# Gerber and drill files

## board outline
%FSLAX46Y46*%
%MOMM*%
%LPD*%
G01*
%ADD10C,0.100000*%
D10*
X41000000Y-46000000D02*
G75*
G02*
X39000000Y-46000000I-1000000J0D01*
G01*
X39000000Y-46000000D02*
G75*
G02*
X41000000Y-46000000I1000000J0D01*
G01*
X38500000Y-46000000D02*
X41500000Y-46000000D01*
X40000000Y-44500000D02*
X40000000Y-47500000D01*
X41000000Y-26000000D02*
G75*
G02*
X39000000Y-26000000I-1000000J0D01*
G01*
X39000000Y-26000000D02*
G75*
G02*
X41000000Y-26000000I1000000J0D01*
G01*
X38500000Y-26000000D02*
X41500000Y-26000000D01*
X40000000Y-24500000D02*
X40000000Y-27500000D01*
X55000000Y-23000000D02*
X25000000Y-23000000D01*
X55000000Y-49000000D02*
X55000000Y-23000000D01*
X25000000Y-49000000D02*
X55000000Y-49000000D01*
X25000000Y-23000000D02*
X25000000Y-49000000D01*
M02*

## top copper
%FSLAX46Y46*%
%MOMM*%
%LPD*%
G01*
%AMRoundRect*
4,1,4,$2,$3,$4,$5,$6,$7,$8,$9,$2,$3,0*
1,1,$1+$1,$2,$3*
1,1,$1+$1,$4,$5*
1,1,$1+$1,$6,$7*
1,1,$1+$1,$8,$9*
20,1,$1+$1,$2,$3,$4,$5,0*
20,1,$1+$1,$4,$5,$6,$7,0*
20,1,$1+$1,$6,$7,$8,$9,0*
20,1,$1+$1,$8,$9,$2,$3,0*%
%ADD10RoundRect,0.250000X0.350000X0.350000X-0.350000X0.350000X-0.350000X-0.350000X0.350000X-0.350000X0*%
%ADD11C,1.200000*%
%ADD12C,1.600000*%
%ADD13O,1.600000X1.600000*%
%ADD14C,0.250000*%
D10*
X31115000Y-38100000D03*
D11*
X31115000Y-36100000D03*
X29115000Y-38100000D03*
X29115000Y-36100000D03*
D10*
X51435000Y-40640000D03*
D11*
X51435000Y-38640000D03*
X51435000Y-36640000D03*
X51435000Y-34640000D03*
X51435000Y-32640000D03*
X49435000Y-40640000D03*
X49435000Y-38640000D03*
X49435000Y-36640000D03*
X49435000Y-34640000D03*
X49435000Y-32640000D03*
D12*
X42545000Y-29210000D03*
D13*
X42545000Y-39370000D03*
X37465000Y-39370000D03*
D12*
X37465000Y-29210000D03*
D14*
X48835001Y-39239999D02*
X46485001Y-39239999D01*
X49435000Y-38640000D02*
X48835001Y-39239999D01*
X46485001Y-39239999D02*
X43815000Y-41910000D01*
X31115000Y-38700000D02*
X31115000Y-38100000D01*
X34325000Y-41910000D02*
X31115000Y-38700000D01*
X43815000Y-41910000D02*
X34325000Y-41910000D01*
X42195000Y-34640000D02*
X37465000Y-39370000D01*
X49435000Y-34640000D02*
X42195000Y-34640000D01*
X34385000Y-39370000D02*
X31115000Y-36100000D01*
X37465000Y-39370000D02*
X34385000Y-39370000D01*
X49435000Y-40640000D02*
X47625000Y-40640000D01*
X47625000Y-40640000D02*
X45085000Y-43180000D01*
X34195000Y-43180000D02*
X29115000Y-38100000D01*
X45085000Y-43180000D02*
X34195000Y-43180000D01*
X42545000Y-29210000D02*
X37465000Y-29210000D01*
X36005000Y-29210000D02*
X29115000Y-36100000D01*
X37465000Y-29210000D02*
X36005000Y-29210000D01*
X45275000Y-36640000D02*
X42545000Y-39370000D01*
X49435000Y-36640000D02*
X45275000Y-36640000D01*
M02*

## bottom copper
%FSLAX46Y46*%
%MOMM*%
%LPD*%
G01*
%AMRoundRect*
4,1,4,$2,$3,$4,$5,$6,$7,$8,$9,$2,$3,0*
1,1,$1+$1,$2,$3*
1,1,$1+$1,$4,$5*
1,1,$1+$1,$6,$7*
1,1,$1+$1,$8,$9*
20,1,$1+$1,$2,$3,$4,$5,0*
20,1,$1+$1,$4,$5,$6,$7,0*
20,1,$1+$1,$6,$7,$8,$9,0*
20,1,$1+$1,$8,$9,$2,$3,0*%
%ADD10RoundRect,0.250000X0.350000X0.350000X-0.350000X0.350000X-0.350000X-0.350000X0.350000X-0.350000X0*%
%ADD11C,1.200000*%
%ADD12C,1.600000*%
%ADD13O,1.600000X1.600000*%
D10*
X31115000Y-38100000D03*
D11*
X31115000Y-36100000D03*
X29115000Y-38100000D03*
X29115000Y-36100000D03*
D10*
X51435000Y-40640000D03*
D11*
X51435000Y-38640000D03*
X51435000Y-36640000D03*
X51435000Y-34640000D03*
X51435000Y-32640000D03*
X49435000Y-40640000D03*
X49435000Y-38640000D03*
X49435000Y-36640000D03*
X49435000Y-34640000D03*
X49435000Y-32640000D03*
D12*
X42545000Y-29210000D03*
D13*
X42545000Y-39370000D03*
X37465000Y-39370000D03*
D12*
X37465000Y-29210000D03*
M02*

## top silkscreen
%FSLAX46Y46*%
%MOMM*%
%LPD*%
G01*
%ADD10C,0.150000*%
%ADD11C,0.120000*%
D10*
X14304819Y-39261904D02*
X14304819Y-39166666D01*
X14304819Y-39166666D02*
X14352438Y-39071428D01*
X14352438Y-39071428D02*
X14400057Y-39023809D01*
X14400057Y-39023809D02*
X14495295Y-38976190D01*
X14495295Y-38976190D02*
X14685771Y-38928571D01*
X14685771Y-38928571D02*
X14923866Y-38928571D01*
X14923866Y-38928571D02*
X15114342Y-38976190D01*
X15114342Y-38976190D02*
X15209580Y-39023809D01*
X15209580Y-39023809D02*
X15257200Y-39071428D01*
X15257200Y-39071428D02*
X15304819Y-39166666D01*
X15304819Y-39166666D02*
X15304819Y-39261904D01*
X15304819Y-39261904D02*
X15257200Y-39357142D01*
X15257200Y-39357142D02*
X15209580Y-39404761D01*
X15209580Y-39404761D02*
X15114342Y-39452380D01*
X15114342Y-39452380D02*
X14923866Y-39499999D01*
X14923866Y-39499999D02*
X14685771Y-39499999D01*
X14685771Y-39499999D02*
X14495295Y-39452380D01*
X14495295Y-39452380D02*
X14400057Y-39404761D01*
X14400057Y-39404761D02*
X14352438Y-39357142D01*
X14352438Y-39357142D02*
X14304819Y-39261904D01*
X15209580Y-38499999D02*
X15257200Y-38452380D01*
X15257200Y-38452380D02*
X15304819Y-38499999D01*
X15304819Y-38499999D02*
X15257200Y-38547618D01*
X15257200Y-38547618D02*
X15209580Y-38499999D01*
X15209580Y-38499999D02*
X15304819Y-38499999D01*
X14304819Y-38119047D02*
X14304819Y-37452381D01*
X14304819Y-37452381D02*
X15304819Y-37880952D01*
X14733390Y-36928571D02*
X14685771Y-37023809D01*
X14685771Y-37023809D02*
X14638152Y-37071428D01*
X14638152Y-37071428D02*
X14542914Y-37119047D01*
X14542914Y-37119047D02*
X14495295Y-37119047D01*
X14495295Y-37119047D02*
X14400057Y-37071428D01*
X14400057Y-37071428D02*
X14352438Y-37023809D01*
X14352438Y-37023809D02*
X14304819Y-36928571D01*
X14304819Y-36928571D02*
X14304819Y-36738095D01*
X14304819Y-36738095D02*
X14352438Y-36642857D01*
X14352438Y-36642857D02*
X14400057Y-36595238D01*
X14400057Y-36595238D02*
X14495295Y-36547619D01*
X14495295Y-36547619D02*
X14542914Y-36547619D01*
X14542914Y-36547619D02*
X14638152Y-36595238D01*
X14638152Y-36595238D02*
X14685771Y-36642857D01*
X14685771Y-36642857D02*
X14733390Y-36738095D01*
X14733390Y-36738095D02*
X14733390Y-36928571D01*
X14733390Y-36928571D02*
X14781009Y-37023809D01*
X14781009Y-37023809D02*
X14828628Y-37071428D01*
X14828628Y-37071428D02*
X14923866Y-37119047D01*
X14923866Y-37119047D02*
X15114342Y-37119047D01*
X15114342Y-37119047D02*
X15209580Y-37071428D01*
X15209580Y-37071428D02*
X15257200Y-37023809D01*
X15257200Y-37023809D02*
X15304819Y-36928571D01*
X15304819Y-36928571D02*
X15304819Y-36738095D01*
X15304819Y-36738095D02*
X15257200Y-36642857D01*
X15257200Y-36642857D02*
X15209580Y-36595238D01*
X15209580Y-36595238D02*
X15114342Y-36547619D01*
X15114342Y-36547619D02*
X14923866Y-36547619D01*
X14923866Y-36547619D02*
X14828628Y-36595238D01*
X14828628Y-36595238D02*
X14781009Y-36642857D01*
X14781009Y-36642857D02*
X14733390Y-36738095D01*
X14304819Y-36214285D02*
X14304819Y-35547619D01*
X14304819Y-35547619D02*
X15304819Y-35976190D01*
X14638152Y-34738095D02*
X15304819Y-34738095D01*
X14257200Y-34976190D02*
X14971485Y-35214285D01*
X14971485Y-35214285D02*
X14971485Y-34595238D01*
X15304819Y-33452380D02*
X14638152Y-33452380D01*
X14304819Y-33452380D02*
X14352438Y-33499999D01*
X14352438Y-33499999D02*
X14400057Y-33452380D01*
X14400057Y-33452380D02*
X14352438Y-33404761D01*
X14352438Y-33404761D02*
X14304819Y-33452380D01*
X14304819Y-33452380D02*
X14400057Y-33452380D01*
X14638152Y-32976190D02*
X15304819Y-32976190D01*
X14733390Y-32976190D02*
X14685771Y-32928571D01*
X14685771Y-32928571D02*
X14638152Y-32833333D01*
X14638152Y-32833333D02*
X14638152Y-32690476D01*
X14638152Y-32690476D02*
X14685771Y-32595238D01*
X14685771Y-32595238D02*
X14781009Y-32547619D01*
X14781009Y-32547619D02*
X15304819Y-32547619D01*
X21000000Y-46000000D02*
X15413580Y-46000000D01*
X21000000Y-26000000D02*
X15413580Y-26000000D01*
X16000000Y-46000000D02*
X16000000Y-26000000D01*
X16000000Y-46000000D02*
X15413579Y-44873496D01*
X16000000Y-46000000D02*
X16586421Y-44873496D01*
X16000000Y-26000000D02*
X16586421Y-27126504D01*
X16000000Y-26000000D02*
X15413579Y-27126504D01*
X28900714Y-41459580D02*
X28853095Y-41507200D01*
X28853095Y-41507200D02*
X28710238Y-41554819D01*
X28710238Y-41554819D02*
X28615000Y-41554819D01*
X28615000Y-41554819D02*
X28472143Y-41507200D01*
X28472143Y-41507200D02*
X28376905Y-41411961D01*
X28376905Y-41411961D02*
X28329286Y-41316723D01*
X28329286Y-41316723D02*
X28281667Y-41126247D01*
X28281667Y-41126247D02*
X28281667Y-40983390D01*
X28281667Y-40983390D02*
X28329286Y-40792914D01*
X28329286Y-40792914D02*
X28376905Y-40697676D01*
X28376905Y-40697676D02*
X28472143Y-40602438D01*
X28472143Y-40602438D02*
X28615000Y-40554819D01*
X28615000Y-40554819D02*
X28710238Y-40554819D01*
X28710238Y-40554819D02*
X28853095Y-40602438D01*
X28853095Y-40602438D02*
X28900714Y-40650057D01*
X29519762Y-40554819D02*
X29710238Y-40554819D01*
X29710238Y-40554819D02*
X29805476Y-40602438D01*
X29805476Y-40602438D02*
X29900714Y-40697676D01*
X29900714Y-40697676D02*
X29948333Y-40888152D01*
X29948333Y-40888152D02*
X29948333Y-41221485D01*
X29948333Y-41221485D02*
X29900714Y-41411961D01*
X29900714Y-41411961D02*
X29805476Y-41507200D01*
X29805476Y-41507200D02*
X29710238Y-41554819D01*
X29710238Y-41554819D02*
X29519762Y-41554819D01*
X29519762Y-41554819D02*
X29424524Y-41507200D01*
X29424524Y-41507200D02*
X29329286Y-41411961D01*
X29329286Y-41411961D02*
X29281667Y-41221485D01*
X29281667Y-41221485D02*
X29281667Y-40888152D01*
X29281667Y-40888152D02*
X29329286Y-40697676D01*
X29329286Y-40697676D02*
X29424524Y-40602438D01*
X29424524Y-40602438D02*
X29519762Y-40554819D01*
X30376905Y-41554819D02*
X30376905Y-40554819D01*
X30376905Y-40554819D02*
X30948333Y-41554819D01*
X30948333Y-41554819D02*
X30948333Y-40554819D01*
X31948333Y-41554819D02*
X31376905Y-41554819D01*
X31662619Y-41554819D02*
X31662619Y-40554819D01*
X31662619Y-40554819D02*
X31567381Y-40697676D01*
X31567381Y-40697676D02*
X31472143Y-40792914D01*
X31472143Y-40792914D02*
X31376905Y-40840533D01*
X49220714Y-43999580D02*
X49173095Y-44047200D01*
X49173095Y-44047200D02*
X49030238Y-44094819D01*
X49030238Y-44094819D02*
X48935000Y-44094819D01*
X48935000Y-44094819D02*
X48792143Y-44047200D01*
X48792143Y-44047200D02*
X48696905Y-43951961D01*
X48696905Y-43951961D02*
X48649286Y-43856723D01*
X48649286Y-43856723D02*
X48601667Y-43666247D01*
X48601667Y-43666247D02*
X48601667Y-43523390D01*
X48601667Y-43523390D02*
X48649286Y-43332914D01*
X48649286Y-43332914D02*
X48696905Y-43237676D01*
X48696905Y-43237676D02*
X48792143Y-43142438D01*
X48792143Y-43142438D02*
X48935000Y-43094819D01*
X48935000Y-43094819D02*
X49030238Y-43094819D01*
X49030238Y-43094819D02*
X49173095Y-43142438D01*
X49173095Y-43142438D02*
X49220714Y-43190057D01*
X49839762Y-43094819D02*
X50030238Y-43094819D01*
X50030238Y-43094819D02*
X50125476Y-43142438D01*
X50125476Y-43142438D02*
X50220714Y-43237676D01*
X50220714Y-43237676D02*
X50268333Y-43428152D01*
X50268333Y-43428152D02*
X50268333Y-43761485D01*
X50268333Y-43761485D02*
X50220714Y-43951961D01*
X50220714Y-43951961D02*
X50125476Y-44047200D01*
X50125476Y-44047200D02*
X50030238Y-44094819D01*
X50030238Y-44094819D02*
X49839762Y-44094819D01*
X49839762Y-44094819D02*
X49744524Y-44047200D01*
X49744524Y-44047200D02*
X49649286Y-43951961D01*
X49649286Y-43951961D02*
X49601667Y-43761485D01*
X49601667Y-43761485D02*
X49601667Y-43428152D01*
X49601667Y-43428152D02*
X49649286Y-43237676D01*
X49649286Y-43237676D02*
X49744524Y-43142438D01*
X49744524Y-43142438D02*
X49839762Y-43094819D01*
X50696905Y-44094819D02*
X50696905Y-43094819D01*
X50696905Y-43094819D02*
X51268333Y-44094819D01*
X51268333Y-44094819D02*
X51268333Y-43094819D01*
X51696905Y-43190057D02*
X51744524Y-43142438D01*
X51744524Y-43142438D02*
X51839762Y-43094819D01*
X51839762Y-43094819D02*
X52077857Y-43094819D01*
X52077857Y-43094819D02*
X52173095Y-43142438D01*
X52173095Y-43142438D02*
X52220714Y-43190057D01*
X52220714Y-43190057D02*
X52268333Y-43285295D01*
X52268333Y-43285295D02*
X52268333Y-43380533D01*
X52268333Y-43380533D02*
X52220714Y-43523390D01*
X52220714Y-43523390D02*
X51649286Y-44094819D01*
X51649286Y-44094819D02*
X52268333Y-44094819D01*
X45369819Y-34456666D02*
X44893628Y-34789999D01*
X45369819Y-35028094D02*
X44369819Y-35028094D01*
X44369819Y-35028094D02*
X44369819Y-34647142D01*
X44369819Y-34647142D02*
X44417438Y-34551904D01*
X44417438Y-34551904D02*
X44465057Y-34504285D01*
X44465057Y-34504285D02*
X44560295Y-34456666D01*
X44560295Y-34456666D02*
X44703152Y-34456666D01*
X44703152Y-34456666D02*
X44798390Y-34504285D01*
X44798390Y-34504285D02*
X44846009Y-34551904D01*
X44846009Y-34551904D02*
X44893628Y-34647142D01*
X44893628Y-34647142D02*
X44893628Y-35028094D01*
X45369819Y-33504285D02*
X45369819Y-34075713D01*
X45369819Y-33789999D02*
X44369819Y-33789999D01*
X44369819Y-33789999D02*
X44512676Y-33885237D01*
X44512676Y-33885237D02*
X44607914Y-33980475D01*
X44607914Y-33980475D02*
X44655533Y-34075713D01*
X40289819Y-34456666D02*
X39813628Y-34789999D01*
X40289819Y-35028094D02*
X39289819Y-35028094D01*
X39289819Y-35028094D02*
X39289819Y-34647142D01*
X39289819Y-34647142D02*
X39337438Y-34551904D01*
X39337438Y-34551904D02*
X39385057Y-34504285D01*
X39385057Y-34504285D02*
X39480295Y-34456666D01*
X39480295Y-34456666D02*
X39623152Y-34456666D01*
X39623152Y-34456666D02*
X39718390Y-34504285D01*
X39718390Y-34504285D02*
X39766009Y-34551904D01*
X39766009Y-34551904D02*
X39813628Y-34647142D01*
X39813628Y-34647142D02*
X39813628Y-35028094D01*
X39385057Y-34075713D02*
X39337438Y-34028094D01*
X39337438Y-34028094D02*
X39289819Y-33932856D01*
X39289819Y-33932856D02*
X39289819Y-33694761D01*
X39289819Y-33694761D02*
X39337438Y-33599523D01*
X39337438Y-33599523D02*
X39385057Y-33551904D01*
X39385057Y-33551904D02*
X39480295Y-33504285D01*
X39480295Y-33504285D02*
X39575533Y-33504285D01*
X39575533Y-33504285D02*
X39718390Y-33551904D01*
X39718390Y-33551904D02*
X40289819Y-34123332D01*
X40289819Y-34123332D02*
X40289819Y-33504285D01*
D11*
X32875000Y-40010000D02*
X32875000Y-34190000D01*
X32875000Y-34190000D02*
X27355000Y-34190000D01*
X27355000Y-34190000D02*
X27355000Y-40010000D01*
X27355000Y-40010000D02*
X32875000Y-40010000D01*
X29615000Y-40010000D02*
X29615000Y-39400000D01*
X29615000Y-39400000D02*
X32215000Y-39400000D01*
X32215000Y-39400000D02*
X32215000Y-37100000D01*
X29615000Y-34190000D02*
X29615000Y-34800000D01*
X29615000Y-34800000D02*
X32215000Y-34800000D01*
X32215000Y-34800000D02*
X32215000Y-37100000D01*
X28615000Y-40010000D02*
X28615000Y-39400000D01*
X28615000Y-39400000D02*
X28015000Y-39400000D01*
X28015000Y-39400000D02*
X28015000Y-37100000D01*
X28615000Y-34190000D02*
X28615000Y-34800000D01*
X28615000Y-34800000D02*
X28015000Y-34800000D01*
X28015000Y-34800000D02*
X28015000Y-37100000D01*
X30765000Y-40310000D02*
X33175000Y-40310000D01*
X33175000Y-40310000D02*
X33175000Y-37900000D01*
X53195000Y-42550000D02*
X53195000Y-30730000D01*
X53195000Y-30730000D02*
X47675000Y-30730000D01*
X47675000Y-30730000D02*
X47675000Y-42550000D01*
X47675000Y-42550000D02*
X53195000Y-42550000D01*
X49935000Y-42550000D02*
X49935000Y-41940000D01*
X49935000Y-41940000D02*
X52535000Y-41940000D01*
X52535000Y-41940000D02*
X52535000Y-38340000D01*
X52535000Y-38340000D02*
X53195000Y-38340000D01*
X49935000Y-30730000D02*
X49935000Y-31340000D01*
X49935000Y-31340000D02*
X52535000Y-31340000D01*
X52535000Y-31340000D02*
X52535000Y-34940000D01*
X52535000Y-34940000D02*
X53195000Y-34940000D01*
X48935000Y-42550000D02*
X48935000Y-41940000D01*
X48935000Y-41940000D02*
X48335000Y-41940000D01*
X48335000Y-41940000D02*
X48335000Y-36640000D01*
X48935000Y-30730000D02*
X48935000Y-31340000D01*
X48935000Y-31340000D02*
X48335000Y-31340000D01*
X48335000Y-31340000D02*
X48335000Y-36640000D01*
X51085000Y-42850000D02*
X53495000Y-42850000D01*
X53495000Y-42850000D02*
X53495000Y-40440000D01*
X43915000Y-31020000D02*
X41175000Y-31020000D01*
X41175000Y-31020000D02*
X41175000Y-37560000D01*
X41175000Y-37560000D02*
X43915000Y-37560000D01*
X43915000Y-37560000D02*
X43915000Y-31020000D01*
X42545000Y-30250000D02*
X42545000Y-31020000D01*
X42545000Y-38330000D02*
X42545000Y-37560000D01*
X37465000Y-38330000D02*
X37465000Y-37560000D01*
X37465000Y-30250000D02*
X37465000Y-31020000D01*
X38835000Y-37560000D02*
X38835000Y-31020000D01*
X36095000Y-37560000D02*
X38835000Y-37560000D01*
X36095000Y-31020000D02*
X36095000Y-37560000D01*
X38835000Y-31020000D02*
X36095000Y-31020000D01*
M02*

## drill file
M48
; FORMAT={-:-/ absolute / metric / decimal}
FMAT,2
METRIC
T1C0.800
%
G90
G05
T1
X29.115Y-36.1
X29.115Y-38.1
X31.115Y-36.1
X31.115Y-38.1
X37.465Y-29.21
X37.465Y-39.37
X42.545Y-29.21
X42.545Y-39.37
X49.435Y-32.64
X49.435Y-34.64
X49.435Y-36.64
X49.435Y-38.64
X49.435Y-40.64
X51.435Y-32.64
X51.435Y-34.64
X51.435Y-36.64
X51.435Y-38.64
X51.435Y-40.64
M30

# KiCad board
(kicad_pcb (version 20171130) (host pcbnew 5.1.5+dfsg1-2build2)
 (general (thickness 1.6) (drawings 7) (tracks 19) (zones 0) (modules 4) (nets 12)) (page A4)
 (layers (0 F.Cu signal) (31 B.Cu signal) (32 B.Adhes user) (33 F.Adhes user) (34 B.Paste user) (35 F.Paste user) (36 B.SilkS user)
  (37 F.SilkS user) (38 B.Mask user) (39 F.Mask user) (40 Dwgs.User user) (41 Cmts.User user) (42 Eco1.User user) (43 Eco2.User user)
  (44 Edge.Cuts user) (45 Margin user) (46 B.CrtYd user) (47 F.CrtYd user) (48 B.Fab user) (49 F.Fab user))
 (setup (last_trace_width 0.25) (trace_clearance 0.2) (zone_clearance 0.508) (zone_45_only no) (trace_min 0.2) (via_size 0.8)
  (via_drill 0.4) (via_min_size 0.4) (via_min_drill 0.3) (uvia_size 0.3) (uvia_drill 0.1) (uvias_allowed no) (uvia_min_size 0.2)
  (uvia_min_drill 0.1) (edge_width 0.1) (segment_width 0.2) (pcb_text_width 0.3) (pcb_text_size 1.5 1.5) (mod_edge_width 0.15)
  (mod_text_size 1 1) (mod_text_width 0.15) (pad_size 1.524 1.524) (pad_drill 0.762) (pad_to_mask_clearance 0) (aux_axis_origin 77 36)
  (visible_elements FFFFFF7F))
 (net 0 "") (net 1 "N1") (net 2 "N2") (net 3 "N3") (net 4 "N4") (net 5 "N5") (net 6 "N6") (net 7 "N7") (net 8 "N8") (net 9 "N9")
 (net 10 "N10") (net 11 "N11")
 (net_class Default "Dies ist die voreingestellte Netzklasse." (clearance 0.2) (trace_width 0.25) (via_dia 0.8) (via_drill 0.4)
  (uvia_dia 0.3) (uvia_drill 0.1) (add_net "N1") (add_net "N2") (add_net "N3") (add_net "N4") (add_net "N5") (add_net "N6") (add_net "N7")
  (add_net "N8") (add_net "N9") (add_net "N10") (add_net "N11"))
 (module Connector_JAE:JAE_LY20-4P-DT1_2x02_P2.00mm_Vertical (layer F.Cu) (at 31.115 38.1 180)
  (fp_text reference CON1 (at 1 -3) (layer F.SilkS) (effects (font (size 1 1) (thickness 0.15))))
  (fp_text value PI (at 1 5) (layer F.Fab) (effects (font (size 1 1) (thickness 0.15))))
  (fp_line (start -1.76 -1.91) (end -1.76 3.91) (layer F.SilkS) (width 0.12))
  (fp_line (start -1.76 3.91) (end 3.76 3.91) (layer F.SilkS) (width 0.12))
  (fp_line (start 3.76 3.91) (end 3.76 -1.91) (layer F.SilkS) (width 0.12))
  (fp_line (start 3.76 -1.91) (end -1.76 -1.91) (layer F.SilkS) (width 0.12))
  (fp_line (start 1.5 -1.91) (end 1.5 -1.3) (layer F.SilkS) (width 0.12))
  (fp_line (start 1.5 -1.3) (end -1.1 -1.3) (layer F.SilkS) (width 0.12))
  (fp_line (start -1.1 -1.3) (end -1.1 1) (layer F.SilkS) (width 0.12))
  (fp_line (start 1.5 3.91) (end 1.5 3.3) (layer F.SilkS) (width 0.12))
  (fp_line (start 1.5 3.3) (end -1.1 3.3) (layer F.SilkS) (width 0.12))
  (fp_line (start -1.1 3.3) (end -1.1 1) (layer F.SilkS) (width 0.12))
  (fp_line (start 2.5 -1.91) (end 2.5 -1.3) (layer F.SilkS) (width 0.12))
  (fp_line (start 2.5 -1.3) (end 3.1 -1.3) (layer F.SilkS) (width 0.12))
  (fp_line (start 3.1 -1.3) (end 3.1 1) (layer F.SilkS) (width 0.12))
  (fp_line (start 2.5 3.91) (end 2.5 3.3) (layer F.SilkS) (width 0.12))
  (fp_line (start 2.5 3.3) (end 3.1 3.3) (layer F.SilkS) (width 0.12))
  (fp_line (start 3.1 3.3) (end 3.1 1) (layer F.SilkS) (width 0.12))
  (fp_line (start 0.35 -2.21) (end -2.06 -2.21) (layer F.SilkS) (width 0.12))
  (fp_line (start -2.06 -2.21) (end -2.06 0.2) (layer F.SilkS) (width 0.12))
  (pad a1 thru_hole roundrect (at 0 0 180) (size 1.2 1.2) (drill 0.8) (layers *.Cu *.Mask) (roundrect_rratio 0.208333) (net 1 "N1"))
  (pad a2 thru_hole circle (at 0 2 180) (size 1.2 1.2) (drill 0.8) (layers *.Cu *.Mask) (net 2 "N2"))
  (pad b1 thru_hole circle (at 2 0 180) (size 1.2 1.2) (drill 0.8) (layers *.Cu *.Mask) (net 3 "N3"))
  (pad b2 thru_hole circle (at 2 2 180) (size 1.2 1.2) (drill 0.8) (layers *.Cu *.Mask) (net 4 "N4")))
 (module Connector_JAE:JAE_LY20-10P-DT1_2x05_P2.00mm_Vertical (layer F.Cu) (at 51.435 40.64 180)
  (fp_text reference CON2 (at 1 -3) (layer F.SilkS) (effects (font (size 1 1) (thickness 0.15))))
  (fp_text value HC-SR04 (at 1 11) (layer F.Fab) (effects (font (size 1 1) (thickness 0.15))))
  (fp_line (start -1.76 -1.91) (end -1.76 9.91) (layer F.SilkS) (width 0.12))
  (fp_line (start -1.76 9.91) (end 3.76 9.91) (layer F.SilkS) (width 0.12))
  (fp_line (start 3.76 9.91) (end 3.76 -1.91) (layer F.SilkS) (width 0.12))
  (fp_line (start 3.76 -1.91) (end -1.76 -1.91) (layer F.SilkS) (width 0.12))
  (fp_line (start 1.5 -1.91) (end 1.5 -1.3) (layer F.SilkS) (width 0.12))
  (fp_line (start 1.5 -1.3) (end -1.1 -1.3) (layer F.SilkS) (width 0.12))
  (fp_line (start -1.1 -1.3) (end -1.1 2.3) (layer F.SilkS) (width 0.12))
  (fp_line (start -1.1 2.3) (end -1.76 2.3) (layer F.SilkS) (width 0.12))
  (fp_line (start 1.5 9.91) (end 1.5 9.3) (layer F.SilkS) (width 0.12))
  (fp_line (start 1.5 9.3) (end -1.1 9.3) (layer F.SilkS) (width 0.12))
  (fp_line (start -1.1 9.3) (end -1.1 5.7) (layer F.SilkS) (width 0.12))
  (fp_line (start -1.1 5.7) (end -1.76 5.7) (layer F.SilkS) (width 0.12))
  (fp_line (start 2.5 -1.91) (end 2.5 -1.3) (layer F.SilkS) (width 0.12))
  (fp_line (start 2.5 -1.3) (end 3.1 -1.3) (layer F.SilkS) (width 0.12))
  (fp_line (start 3.1 -1.3) (end 3.1 4) (layer F.SilkS) (width 0.12))
  (fp_line (start 2.5 9.91) (end 2.5 9.3) (layer F.SilkS) (width 0.12))
  (fp_line (start 2.5 9.3) (end 3.1 9.3) (layer F.SilkS) (width 0.12))
  (fp_line (start 3.1 9.3) (end 3.1 4) (layer F.SilkS) (width 0.12))
  (fp_line (start 0.35 -2.21) (end -2.06 -2.21) (layer F.SilkS) (width 0.12))
  (fp_line (start -2.06 -2.21) (end -2.06 0.2) (layer F.SilkS) (width 0.12))
  (pad a1 thru_hole roundrect (at 0 0 180) (size 1.2 1.2) (drill 0.8) (layers *.Cu *.Mask) (roundrect_rratio 0.208333) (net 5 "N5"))
  (pad a2 thru_hole circle (at 0 2 180) (size 1.2 1.2) (drill 0.8) (layers *.Cu *.Mask) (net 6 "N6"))
  (pad a3 thru_hole circle (at 0 4 180) (size 1.2 1.2) (drill 0.8) (layers *.Cu *.Mask) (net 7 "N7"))
  (pad a4 thru_hole circle (at 0 6 180) (size 1.2 1.2) (drill 0.8) (layers *.Cu *.Mask) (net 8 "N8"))
  (pad a5 thru_hole circle (at 0 8 180) (size 1.2 1.2) (drill 0.8) (layers *.Cu *.Mask) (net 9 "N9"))
  (pad b1 thru_hole circle (at 2 0 180) (size 1.2 1.2) (drill 0.8) (layers *.Cu *.Mask) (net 3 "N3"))
  (pad b2 thru_hole circle (at 2 2 180) (size 1.2 1.2) (drill 0.8) (layers *.Cu *.Mask) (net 1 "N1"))
  (pad b3 thru_hole circle (at 2 4 180) (size 1.2 1.2) (drill 0.8) (layers *.Cu *.Mask) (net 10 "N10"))
  (pad b4 thru_hole circle (at 2 6 180) (size 1.2 1.2) (drill 0.8) (layers *.Cu *.Mask) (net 2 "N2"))
  (pad b5 thru_hole circle (at 2 8 180) (size 1.2 1.2) (drill 0.8) (layers *.Cu *.Mask) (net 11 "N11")))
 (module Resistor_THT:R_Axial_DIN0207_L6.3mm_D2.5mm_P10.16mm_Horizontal (layer F.Cu) (at 42.545 29.21 270)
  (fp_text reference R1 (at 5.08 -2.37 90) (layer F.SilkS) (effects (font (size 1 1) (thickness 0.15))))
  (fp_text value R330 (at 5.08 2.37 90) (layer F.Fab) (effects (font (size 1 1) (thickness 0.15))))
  (fp_line (start 1.81 -1.37) (end 1.81 1.37) (layer F.SilkS) (width 0.12))
  (fp_line (start 1.81 1.37) (end 8.35 1.37) (layer F.SilkS) (width 0.12))
  (fp_line (start 8.35 1.37) (end 8.35 -1.37) (layer F.SilkS) (width 0.12))
  (fp_line (start 8.35 -1.37) (end 1.81 -1.37) (layer F.SilkS) (width 0.12))
  (fp_line (start 1.04 0) (end 1.81 0) (layer F.SilkS) (width 0.12))
  (fp_line (start 9.12 0) (end 8.35 0) (layer F.SilkS) (width 0.12))
  (pad 1 thru_hole circle (at 0 0 270) (size 1.6 1.6) (drill 0.8) (layers *.Cu *.Mask) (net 4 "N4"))
  (pad 2 thru_hole oval (at 10.16 0 270) (size 1.6 1.6) (drill 0.8) (layers *.Cu *.Mask) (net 10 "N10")))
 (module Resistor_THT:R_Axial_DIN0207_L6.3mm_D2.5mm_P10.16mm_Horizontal (layer F.Cu) (at 37.465 29.21 270)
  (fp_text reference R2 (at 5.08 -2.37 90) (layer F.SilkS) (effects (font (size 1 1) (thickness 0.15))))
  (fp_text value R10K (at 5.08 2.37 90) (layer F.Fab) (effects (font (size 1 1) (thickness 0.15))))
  (fp_line (start 9.12 0) (end 8.35 0) (layer F.SilkS) (width 0.12))
  (fp_line (start 1.04 0) (end 1.81 0) (layer F.SilkS) (width 0.12))
  (fp_line (start 8.35 -1.37) (end 1.81 -1.37) (layer F.SilkS) (width 0.12))
  (fp_line (start 8.35 1.37) (end 8.35 -1.37) (layer F.SilkS) (width 0.12))
  (fp_line (start 1.81 1.37) (end 8.35 1.37) (layer F.SilkS) (width 0.12))
  (fp_line (start 1.81 -1.37) (end 1.81 1.37) (layer F.SilkS) (width 0.12))
  (pad 2 thru_hole oval (at 10.16 0 270) (size 1.6 1.6) (drill 0.8) (layers *.Cu *.Mask) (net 2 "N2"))
  (pad 1 thru_hole circle (at 0 0 270) (size 1.6 1.6) (drill 0.8) (layers *.Cu *.Mask) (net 4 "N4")))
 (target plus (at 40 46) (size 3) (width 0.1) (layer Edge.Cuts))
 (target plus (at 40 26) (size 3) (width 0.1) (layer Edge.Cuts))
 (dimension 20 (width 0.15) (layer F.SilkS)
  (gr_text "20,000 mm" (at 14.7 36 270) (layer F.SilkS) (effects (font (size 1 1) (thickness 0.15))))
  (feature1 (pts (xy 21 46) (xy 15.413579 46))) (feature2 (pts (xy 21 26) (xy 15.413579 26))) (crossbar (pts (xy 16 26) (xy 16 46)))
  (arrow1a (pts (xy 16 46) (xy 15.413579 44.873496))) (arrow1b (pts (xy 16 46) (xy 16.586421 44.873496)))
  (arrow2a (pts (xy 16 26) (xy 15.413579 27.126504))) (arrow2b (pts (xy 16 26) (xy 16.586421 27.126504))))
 (gr_line (start 55 23) (end 25 23) (layer Edge.Cuts) (width 0.1))
 (gr_line (start 55 49) (end 55 23) (layer Edge.Cuts) (width 0.1))
 (gr_line (start 25 49) (end 55 49) (layer Edge.Cuts) (width 0.1))
 (gr_line (start 25 23) (end 25 49) (layer Edge.Cuts) (width 0.1))
 (segment (start 48.835001 39.239999) (end 46.485001 39.239999) (width 0.25) (layer F.Cu) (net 1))
 (segment (start 49.435 38.64) (end 48.835001 39.239999) (width 0.25) (layer F.Cu) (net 1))
 (segment (start 46.485001 39.239999) (end 43.815 41.91) (width 0.25) (layer F.Cu) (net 1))
 (segment (start 31.115 38.7) (end 31.115 38.1) (width 0.25) (layer F.Cu) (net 1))
 (segment (start 34.325 41.91) (end 31.115 38.7) (width 0.25) (layer F.Cu) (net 1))
 (segment (start 43.815 41.91) (end 34.325 41.91) (width 0.25) (layer F.Cu) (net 1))
 (segment (start 42.195 34.64) (end 37.465 39.37) (width 0.25) (layer F.Cu) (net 2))
 (segment (start 49.435 34.64) (end 42.195 34.64) (width 0.25) (layer F.Cu) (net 2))
 (segment (start 34.385 39.37) (end 31.115 36.1) (width 0.25) (layer F.Cu) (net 2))
 (segment (start 37.465 39.37) (end 34.385 39.37) (width 0.25) (layer F.Cu) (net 2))
 (segment (start 49.435 40.64) (end 47.625 40.64) (width 0.25) (layer F.Cu) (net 3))
 (segment (start 47.625 40.64) (end 45.085 43.18) (width 0.25) (layer F.Cu) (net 3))
 (segment (start 34.195 43.18) (end 29.115 38.1) (width 0.25) (layer F.Cu) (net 3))
 (segment (start 45.085 43.18) (end 34.195 43.18) (width 0.25) (layer F.Cu) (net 3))
 (segment (start 42.545 29.21) (end 37.465 29.21) (width 0.25) (layer F.Cu) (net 4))
 (segment (start 36.005 29.21) (end 29.115 36.1) (width 0.25) (layer F.Cu) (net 4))
 (segment (start 37.465 29.21) (end 36.005 29.21) (width 0.25) (layer F.Cu) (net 4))
 (segment (start 45.275 36.64) (end 42.545 39.37) (width 0.25) (layer F.Cu) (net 10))
 (segment (start 49.435 36.64) (end 45.275 36.64) (width 0.25) (layer F.Cu) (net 10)))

